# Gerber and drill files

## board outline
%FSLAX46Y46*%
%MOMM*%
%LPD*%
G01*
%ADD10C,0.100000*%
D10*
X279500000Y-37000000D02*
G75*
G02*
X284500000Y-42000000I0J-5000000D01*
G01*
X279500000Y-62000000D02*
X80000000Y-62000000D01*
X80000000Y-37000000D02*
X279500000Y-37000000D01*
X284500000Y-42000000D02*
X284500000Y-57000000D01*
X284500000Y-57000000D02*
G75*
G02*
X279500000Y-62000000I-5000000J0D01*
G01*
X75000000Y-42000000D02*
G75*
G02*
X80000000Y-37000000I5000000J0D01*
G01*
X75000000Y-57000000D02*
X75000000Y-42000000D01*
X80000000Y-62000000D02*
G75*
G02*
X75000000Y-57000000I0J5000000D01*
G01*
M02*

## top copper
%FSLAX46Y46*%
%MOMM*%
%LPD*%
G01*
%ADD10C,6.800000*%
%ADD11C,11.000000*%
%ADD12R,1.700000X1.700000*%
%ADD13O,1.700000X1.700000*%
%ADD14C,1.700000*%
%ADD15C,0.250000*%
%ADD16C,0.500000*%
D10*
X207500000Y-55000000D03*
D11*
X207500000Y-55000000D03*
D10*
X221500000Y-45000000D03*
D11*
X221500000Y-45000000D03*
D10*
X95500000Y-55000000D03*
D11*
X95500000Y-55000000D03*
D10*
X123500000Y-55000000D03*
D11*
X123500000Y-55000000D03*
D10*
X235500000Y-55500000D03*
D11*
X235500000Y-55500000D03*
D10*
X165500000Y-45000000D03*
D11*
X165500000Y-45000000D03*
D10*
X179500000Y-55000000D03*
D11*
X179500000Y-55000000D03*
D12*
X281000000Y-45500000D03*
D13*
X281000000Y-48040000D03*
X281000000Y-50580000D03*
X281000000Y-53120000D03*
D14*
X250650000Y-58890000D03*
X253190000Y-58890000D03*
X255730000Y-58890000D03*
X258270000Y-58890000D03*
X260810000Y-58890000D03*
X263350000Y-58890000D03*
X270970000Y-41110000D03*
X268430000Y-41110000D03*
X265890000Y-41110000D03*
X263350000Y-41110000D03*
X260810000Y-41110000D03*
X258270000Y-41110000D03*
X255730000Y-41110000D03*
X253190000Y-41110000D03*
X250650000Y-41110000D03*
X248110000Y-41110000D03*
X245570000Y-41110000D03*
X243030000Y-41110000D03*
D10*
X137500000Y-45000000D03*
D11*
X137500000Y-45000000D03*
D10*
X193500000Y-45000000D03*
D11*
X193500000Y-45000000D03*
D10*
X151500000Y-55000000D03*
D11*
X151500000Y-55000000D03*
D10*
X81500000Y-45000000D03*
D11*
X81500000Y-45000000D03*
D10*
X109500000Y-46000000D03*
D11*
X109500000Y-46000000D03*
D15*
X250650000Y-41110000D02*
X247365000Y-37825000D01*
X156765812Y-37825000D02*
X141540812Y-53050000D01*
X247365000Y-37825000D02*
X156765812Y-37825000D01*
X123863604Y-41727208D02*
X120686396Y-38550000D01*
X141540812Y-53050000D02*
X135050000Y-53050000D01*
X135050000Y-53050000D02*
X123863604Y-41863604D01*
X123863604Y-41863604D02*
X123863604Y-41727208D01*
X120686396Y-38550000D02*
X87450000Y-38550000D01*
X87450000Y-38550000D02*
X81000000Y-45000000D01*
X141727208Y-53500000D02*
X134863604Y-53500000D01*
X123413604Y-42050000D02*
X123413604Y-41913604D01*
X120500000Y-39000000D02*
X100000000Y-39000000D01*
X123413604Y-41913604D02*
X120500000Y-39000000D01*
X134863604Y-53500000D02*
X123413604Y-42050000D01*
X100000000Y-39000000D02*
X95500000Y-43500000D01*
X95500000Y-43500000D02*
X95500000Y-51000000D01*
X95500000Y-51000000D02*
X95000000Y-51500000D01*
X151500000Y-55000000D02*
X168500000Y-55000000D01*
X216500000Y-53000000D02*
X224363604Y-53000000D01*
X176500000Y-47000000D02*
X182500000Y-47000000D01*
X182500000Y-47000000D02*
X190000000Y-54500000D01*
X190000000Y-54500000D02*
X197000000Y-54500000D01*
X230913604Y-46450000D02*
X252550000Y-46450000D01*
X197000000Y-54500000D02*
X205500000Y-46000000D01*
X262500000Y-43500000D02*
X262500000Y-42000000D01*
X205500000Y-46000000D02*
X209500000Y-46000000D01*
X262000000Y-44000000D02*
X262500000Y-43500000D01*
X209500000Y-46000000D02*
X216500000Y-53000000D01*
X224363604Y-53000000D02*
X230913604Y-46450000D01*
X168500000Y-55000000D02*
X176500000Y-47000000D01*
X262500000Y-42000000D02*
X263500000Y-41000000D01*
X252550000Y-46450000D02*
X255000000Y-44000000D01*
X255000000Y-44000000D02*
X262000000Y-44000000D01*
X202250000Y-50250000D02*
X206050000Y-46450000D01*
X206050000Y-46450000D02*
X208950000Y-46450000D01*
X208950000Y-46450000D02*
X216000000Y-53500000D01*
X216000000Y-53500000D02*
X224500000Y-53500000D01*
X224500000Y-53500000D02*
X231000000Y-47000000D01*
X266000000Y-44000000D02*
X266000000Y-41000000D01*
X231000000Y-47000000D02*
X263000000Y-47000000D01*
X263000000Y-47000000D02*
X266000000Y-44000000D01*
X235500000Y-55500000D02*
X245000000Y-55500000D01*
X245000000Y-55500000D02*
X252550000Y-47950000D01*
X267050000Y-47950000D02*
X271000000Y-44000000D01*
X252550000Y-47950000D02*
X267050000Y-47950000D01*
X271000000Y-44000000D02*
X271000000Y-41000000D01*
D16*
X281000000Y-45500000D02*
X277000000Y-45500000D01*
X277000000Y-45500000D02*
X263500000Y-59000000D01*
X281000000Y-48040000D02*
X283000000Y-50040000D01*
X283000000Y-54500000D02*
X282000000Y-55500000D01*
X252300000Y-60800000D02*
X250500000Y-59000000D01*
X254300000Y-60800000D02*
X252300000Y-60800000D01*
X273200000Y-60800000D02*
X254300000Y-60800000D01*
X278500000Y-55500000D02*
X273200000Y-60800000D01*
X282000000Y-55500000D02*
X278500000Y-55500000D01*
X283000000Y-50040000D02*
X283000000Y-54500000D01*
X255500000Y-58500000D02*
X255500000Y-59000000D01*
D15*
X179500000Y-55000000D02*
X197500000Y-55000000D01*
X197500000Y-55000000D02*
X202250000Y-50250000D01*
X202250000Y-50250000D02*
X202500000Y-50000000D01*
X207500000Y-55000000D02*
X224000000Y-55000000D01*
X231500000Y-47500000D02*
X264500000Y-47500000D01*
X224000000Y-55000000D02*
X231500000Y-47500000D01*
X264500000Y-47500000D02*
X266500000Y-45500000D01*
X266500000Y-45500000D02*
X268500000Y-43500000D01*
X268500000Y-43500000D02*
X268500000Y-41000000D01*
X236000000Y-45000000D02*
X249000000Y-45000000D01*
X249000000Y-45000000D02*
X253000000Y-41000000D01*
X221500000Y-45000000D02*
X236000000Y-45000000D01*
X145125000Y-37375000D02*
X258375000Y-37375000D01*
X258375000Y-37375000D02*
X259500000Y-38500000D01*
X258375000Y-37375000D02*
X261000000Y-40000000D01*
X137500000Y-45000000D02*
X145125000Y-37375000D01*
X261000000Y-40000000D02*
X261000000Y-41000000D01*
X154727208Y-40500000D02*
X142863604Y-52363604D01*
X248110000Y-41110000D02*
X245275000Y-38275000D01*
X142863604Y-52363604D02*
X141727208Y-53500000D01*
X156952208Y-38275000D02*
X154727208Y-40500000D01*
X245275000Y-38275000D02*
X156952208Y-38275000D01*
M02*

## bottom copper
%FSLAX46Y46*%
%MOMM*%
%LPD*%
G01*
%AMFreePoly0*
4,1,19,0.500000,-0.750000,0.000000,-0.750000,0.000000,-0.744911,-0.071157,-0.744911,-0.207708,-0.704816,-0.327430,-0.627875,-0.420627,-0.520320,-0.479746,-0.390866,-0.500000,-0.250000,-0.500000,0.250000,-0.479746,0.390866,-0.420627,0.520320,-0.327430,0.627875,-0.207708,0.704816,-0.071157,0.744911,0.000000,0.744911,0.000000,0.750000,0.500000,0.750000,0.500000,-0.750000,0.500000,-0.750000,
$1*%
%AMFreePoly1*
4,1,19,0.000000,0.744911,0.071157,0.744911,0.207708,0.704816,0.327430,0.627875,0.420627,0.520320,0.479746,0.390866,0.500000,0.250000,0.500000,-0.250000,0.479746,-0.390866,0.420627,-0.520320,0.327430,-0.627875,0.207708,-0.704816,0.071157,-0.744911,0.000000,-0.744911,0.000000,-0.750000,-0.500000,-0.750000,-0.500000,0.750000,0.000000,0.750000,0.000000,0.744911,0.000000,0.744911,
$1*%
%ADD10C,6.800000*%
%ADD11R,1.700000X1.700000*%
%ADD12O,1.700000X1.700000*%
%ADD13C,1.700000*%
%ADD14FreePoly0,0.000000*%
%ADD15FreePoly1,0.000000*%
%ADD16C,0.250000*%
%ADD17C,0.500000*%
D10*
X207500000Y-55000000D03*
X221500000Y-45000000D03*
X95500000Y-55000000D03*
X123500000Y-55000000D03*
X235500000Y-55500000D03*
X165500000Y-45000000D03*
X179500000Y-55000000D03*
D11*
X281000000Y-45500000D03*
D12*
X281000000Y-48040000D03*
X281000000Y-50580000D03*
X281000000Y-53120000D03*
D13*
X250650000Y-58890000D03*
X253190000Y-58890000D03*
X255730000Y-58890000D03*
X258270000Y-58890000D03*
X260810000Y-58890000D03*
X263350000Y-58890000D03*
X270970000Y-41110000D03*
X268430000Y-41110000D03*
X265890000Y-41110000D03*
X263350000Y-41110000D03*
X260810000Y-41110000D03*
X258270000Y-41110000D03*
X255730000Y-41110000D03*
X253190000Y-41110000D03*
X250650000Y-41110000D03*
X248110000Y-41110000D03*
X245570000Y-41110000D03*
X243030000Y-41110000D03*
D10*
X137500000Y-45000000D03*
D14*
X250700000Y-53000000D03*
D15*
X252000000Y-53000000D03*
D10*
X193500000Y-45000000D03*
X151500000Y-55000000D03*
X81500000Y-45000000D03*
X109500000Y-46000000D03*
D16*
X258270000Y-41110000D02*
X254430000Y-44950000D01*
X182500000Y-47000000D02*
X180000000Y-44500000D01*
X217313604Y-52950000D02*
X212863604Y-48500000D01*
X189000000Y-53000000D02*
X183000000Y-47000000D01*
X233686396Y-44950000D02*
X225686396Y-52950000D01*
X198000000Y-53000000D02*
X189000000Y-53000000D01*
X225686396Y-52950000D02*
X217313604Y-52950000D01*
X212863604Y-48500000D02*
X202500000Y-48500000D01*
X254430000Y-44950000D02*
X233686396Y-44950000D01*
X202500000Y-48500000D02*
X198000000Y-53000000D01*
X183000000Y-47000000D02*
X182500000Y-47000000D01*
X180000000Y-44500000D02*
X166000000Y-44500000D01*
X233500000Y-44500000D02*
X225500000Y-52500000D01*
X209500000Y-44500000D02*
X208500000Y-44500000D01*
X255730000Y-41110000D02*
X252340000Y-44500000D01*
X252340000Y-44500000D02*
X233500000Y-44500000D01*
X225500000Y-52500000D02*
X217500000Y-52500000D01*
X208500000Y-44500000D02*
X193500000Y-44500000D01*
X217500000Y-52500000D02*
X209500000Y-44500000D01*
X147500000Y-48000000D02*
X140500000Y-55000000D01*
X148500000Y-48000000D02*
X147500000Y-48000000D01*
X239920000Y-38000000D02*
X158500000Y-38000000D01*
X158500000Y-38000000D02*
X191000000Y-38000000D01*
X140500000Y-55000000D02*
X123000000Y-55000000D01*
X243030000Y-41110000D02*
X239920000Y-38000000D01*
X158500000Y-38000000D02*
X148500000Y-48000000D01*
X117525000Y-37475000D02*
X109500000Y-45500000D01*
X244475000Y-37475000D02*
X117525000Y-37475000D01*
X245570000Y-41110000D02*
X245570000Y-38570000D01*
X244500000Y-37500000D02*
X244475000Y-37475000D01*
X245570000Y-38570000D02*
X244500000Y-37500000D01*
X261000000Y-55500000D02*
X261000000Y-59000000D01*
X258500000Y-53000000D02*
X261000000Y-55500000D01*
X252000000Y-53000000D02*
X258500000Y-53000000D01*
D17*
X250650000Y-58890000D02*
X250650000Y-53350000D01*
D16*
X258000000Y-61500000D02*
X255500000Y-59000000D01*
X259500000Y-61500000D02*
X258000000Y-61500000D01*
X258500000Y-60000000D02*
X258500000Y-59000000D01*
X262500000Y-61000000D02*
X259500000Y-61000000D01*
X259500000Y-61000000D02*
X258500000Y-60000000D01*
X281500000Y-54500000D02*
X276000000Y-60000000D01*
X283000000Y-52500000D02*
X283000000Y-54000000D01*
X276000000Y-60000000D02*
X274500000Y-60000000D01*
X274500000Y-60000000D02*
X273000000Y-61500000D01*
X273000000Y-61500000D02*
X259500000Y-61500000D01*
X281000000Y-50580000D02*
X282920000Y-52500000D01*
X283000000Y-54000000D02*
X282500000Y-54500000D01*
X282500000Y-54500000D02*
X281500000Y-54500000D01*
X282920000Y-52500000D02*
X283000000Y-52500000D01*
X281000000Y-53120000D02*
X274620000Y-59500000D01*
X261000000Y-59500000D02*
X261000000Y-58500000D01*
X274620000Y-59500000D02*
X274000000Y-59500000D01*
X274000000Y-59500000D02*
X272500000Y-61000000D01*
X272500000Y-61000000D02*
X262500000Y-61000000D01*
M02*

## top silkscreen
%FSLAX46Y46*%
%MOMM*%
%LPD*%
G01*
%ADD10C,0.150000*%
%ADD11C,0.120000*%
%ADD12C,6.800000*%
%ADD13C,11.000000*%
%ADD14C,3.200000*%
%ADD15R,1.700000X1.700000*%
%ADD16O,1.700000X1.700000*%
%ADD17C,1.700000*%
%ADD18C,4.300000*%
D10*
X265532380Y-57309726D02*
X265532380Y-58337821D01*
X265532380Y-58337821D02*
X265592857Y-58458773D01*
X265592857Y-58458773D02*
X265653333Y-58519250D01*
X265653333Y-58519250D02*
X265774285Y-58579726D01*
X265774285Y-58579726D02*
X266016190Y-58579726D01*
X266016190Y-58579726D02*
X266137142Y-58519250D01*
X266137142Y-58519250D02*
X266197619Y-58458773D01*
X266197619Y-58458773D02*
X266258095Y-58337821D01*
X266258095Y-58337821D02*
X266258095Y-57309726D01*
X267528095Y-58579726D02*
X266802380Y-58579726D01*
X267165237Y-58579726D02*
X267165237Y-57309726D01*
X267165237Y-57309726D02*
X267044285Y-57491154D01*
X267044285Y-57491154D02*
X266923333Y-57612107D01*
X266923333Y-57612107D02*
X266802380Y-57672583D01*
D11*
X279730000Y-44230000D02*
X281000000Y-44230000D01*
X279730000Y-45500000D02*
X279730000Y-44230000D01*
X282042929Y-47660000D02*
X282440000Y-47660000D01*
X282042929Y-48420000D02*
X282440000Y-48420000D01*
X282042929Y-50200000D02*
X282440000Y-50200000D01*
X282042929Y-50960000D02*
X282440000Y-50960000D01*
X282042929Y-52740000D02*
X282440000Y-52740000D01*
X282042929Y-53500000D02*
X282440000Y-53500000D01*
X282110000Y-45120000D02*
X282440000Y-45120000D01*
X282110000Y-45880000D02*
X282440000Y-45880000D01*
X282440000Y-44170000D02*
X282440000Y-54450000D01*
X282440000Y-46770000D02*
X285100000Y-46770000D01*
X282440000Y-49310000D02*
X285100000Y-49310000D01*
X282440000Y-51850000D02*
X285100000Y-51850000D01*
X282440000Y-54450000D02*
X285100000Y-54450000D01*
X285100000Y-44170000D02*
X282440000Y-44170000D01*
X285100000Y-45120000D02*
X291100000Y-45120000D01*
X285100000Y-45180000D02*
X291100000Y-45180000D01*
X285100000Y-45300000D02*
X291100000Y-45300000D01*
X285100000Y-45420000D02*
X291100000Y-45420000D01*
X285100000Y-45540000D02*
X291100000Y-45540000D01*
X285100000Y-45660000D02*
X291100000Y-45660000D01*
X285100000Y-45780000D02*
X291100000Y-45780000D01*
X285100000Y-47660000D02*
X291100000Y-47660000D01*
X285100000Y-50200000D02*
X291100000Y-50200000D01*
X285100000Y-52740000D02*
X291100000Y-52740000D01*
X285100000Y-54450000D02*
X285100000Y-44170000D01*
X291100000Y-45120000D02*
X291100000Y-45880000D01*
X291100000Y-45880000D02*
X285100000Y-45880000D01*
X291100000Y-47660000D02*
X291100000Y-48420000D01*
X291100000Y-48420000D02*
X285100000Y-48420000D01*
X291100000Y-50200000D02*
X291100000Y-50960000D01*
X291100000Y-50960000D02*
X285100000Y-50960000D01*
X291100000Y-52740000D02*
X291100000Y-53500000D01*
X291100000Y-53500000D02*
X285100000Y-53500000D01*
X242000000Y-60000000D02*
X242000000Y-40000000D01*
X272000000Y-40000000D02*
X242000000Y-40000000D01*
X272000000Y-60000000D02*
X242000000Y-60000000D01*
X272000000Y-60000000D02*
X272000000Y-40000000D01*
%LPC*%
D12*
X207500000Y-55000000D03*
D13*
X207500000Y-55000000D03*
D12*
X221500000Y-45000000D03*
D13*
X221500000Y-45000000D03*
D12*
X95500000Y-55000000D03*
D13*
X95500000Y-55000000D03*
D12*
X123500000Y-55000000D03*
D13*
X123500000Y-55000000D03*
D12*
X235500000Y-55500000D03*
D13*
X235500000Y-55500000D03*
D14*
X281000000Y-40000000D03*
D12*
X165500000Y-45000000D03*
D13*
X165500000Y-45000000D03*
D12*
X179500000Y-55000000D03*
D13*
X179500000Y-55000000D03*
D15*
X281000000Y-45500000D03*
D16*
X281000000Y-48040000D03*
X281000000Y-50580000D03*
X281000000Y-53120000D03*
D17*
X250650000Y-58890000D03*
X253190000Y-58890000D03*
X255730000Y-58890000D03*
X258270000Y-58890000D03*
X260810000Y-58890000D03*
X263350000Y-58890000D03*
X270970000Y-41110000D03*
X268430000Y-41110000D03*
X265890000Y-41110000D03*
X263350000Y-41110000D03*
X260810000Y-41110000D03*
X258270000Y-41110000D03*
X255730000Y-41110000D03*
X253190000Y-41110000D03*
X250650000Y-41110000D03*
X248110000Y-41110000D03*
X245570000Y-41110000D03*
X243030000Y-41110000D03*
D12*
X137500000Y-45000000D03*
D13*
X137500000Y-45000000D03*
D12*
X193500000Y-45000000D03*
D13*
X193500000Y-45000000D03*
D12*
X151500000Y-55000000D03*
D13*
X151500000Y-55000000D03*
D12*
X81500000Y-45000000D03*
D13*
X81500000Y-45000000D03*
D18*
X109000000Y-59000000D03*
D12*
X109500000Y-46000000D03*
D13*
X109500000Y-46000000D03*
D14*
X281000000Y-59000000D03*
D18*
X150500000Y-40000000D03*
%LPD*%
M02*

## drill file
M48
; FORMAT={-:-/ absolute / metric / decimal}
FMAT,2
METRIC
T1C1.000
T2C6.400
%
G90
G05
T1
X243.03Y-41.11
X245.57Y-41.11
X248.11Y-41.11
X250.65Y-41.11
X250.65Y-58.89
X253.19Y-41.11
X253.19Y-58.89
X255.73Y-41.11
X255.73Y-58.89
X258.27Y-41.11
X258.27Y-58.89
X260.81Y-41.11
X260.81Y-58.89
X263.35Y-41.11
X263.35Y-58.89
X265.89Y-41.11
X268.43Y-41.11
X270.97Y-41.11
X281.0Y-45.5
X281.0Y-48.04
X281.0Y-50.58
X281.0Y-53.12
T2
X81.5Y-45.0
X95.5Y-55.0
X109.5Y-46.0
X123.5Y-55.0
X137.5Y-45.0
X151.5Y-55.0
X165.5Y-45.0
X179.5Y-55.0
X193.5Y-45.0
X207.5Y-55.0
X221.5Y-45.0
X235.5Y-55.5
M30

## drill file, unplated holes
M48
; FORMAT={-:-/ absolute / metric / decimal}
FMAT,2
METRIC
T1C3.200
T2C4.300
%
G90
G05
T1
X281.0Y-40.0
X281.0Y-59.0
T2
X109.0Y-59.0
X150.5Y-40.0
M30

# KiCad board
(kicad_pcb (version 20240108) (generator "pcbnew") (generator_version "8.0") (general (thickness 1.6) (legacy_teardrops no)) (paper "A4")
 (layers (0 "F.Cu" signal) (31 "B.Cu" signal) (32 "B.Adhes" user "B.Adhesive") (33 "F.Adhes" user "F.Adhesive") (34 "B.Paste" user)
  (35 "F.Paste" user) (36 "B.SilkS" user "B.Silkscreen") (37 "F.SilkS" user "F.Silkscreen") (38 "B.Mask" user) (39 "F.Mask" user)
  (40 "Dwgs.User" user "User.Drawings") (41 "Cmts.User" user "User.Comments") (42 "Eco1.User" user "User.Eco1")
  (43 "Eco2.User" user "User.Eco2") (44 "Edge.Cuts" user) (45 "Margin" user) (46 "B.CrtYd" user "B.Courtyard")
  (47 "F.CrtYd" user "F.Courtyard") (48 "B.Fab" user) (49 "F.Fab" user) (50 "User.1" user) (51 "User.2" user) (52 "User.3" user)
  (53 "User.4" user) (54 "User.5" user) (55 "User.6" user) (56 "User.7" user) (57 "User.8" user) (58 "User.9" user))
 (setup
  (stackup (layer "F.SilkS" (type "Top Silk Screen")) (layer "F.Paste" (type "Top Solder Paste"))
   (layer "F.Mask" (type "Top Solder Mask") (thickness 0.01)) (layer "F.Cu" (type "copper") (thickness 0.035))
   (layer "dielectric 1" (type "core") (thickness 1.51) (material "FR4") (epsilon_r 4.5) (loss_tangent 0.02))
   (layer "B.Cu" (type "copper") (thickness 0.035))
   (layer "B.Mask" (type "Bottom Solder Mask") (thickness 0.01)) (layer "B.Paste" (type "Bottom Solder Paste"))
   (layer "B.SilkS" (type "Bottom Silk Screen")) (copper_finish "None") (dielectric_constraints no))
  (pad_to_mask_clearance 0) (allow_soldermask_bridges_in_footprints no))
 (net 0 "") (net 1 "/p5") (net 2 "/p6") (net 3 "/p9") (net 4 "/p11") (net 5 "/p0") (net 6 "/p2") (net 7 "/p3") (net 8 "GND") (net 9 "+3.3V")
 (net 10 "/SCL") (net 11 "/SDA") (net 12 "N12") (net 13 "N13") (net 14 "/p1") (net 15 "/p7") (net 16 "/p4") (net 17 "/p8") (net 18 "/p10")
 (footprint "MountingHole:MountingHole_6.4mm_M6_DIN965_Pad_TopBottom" (layer "F.Cu") (at 207.5 55 90)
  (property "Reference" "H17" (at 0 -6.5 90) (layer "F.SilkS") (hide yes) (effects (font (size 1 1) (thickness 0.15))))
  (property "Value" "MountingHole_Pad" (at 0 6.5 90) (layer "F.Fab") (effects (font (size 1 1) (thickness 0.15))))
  (pad "" connect circle (at 0 0 90) (size 11 11) (layers "B.Mask" "Rescue"))
  (pad "1" thru_hole circle (at 0 0 90) (size 6.8 6.8) (drill 6.4) (layers "*.Cu" "*.Mask") (remove_unused_layers no) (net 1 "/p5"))
  (pad "1" connect circle (at 0 0 90) (size 11 11) (layers "F.Cu" "F.Mask") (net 1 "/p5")))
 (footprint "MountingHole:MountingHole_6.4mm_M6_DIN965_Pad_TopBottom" (layer "F.Cu") (at 221.5 45 90)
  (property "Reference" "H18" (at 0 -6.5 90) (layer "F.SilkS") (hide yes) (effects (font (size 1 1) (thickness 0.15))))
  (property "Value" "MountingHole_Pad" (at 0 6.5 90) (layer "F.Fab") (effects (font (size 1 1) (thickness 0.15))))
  (pad "" connect circle (at 0 0 90) (size 11 11) (layers "B.Mask" "Rescue"))
  (pad "1" thru_hole circle (at 0 0 90) (size 6.8 6.8) (drill 6.4) (layers "*.Cu" "*.Mask") (remove_unused_layers no) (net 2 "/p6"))
  (pad "1" connect circle (at 0 0 90) (size 11 11) (layers "F.Cu" "F.Mask") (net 2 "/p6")))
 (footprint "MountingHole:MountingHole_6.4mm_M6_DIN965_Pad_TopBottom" (layer "F.Cu") (at 95.5 55)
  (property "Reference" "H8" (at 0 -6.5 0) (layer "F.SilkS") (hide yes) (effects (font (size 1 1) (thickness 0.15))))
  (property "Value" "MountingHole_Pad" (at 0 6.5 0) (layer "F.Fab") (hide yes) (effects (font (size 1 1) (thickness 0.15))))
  (pad "" connect circle (at 0 0) (size 11 11) (layers "B.Mask" "Rescue"))
  (pad "1" thru_hole circle (at 0 0) (size 6.8 6.8) (drill 6.4) (layers "*.Cu" "*.Mask") (remove_unused_layers no) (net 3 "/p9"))
  (pad "1" connect circle (at 0 0) (size 11 11) (layers "F.Cu" "F.Mask") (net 3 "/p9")))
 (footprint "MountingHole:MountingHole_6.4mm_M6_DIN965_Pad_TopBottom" (layer "F.Cu") (at 123.5 55 90)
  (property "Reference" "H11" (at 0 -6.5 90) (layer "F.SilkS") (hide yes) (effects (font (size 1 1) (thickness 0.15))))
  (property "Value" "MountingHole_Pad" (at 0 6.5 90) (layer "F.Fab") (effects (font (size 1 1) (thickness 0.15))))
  (pad "" connect circle (at 0 0 90) (size 11 11) (layers "B.Mask" "Rescue"))
  (pad "1" thru_hole circle (at 0 0 90) (size 6.8 6.8) (drill 6.4) (layers "*.Cu" "*.Mask") (remove_unused_layers no) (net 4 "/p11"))
  (pad "1" connect circle (at 0 0 90) (size 11 11) (layers "F.Cu" "F.Mask") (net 4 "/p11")))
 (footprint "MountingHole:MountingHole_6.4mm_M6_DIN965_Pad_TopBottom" (layer "F.Cu") (at 235.5 55.5 90)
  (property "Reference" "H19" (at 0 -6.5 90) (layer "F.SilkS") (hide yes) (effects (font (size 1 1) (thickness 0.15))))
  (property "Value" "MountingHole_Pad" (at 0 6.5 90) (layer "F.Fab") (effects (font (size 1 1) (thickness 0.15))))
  (pad "" connect circle (at 0 0 90) (size 11 11) (layers "B.Mask" "Rescue"))
  (pad "1" thru_hole circle (at 0 0 90) (size 6.8 6.8) (drill 6.4) (layers "*.Cu" "*.Mask") (remove_unused_layers no) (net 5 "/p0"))
  (pad "1" connect circle (at 0 0 90) (size 11 11) (layers "F.Cu" "F.Mask") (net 5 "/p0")))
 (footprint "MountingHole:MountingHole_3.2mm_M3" (layer "F.Cu") (at 283.7475 40.08 -90)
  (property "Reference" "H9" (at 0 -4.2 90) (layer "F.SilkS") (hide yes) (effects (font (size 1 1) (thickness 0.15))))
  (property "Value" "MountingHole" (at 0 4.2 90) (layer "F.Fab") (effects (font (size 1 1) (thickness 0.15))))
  (pad "" np_thru_hole circle (at -0.08 2.7475 270) (size 3.2 3.2) (drill 3.2) (layers "F&B.Cu" "*.Mask")))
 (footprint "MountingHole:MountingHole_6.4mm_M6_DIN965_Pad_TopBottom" (layer "F.Cu") (at 165.5 45 90)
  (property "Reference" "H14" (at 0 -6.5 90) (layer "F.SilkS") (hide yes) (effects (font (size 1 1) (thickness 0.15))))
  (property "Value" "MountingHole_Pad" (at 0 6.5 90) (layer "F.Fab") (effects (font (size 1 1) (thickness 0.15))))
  (pad "" connect circle (at 0 0 90) (size 11 11) (layers "B.Mask" "Rescue"))
  (pad "1" thru_hole circle (at 0 0 90) (size 6.8 6.8) (drill 6.4) (layers "*.Cu" "*.Mask") (remove_unused_layers no) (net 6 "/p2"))
  (pad "1" connect circle (at 0 0 90) (size 11 11) (layers "F.Cu" "F.Mask") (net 6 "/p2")))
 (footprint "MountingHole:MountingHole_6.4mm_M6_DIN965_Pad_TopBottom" (layer "F.Cu") (at 179.5 55 90)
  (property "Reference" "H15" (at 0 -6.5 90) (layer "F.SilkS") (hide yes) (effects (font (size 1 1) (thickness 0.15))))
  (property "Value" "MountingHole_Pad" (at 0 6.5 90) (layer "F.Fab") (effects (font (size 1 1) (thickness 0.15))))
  (pad "" connect circle (at 0 0 90) (size 11 11) (layers "B.Mask" "Rescue"))
  (pad "1" thru_hole circle (at 0 0 90) (size 6.8 6.8) (drill 6.4) (layers "*.Cu" "*.Mask") (remove_unused_layers no) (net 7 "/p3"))
  (pad "1" connect circle (at 0 0 90) (size 11 11) (layers "F.Cu" "F.Mask") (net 7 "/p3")))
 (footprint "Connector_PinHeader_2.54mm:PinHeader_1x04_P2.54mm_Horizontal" (layer "F.Cu") (at 281 45.5)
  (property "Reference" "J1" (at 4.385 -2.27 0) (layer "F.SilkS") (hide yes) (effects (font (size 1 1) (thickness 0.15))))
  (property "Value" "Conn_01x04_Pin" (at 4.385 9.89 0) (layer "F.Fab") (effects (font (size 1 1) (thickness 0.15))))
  (fp_line (start -1.27 -1.27) (end 0 -1.27) (stroke (width 0.12) (type solid)) (layer "F.SilkS"))
  (fp_line (start -1.27 0) (end -1.27 -1.27) (stroke (width 0.12) (type solid)) (layer "F.SilkS"))
  (fp_line (start 1.042929 2.16) (end 1.44 2.16) (stroke (width 0.12) (type solid)) (layer "F.SilkS"))
  (fp_line (start 1.042929 2.92) (end 1.44 2.92) (stroke (width 0.12) (type solid)) (layer "F.SilkS"))
  (fp_line (start 1.042929 4.7) (end 1.44 4.7) (stroke (width 0.12) (type solid)) (layer "F.SilkS"))
  (fp_line (start 1.042929 5.46) (end 1.44 5.46) (stroke (width 0.12) (type solid)) (layer "F.SilkS"))
  (fp_line (start 1.042929 7.24) (end 1.44 7.24) (stroke (width 0.12) (type solid)) (layer "F.SilkS"))
  (fp_line (start 1.042929 8) (end 1.44 8) (stroke (width 0.12) (type solid)) (layer "F.SilkS"))
  (fp_line (start 1.11 -0.38) (end 1.44 -0.38) (stroke (width 0.12) (type solid)) (layer "F.SilkS"))
  (fp_line (start 1.11 0.38) (end 1.44 0.38) (stroke (width 0.12) (type solid)) (layer "F.SilkS"))
  (fp_line (start 1.44 -1.33) (end 1.44 8.95) (stroke (width 0.12) (type solid)) (layer "F.SilkS"))
  (fp_line (start 1.44 1.27) (end 4.1 1.27) (stroke (width 0.12) (type solid)) (layer "F.SilkS"))
  (fp_line (start 1.44 3.81) (end 4.1 3.81) (stroke (width 0.12) (type solid)) (layer "F.SilkS"))
  (fp_line (start 1.44 6.35) (end 4.1 6.35) (stroke (width 0.12) (type solid)) (layer "F.SilkS"))
  (fp_line (start 1.44 8.95) (end 4.1 8.95) (stroke (width 0.12) (type solid)) (layer "F.SilkS"))
  (fp_line (start 4.1 -1.33) (end 1.44 -1.33) (stroke (width 0.12) (type solid)) (layer "F.SilkS"))
  (fp_line (start 4.1 -0.38) (end 10.1 -0.38) (stroke (width 0.12) (type solid)) (layer "F.SilkS"))
  (fp_line (start 4.1 -0.32) (end 10.1 -0.32) (stroke (width 0.12) (type solid)) (layer "F.SilkS"))
  (fp_line (start 4.1 -0.2) (end 10.1 -0.2) (stroke (width 0.12) (type solid)) (layer "F.SilkS"))
  (fp_line (start 4.1 -0.08) (end 10.1 -0.08) (stroke (width 0.12) (type solid)) (layer "F.SilkS"))
  (fp_line (start 4.1 0.04) (end 10.1 0.04) (stroke (width 0.12) (type solid)) (layer "F.SilkS"))
  (fp_line (start 4.1 0.16) (end 10.1 0.16) (stroke (width 0.12) (type solid)) (layer "F.SilkS"))
  (fp_line (start 4.1 0.28) (end 10.1 0.28) (stroke (width 0.12) (type solid)) (layer "F.SilkS"))
  (fp_line (start 4.1 2.16) (end 10.1 2.16) (stroke (width 0.12) (type solid)) (layer "F.SilkS"))
  (fp_line (start 4.1 4.7) (end 10.1 4.7) (stroke (width 0.12) (type solid)) (layer "F.SilkS"))
  (fp_line (start 4.1 7.24) (end 10.1 7.24) (stroke (width 0.12) (type solid)) (layer "F.SilkS"))
  (fp_line (start 4.1 8.95) (end 4.1 -1.33) (stroke (width 0.12) (type solid)) (layer "F.SilkS"))
  (fp_line (start 10.1 -0.38) (end 10.1 0.38) (stroke (width 0.12) (type solid)) (layer "F.SilkS"))
  (fp_line (start 10.1 0.38) (end 4.1 0.38) (stroke (width 0.12) (type solid)) (layer "F.SilkS"))
  (fp_line (start 10.1 2.16) (end 10.1 2.92) (stroke (width 0.12) (type solid)) (layer "F.SilkS"))
  (fp_line (start 10.1 2.92) (end 4.1 2.92) (stroke (width 0.12) (type solid)) (layer "F.SilkS"))
  (fp_line (start 10.1 4.7) (end 10.1 5.46) (stroke (width 0.12) (type solid)) (layer "F.SilkS"))
  (fp_line (start 10.1 5.46) (end 4.1 5.46) (stroke (width 0.12) (type solid)) (layer "F.SilkS"))
  (fp_line (start 10.1 7.24) (end 10.1 8) (stroke (width 0.12) (type solid)) (layer "F.SilkS"))
  (fp_line (start 10.1 8) (end 4.1 8) (stroke (width 0.12) (type solid)) (layer "F.SilkS"))
  (pad "1" thru_hole rect (at 0 0) (size 1.7 1.7) (drill 1) (layers "*.Cu" "*.Mask") (remove_unused_layers no) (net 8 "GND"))
  (pad "2" thru_hole oval (at 0 2.54) (size 1.7 1.7) (drill 1) (layers "*.Cu" "*.Mask") (remove_unused_layers no) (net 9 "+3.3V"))
  (pad "3" thru_hole oval (at 0 5.08) (size 1.7 1.7) (drill 1) (layers "*.Cu" "*.Mask") (remove_unused_layers no) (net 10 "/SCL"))
  (pad "4" thru_hole oval (at 0 7.62) (size 1.7 1.7) (drill 1) (layers "*.Cu" "*.Mask") (remove_unused_layers no) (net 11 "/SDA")))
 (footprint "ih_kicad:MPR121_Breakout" (layer "F.Cu") (at 257 50 180)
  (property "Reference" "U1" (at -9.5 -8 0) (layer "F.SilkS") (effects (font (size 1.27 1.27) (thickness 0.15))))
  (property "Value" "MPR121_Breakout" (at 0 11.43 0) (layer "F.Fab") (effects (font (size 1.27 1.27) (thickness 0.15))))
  (fp_line (start 15 -10) (end 15 10) (stroke (width 0.12) (type solid)) (layer "F.SilkS"))
  (fp_line (start -15 10) (end 15 10) (stroke (width 0.12) (type solid)) (layer "F.SilkS"))
  (fp_line (start -15 -10) (end 15 -10) (stroke (width 0.12) (type solid)) (layer "F.SilkS"))
  (fp_line (start -15 -10) (end -15 10) (stroke (width 0.12) (type solid)) (layer "F.SilkS"))
  (pad "1" thru_hole circle (at 6.35 -8.89 180) (size 1.7 1.7) (drill 1) (layers "*.Cu" "*.Mask") (remove_unused_layers no) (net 9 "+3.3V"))
  (pad "2" thru_hole circle (at 3.81 -8.89 180) (size 1.7 1.7) (drill 1) (layers "*.Cu" "*.Mask") (remove_unused_layers no) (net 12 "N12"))
  (pad "3" thru_hole circle (at 1.27 -8.89 180) (size 1.7 1.7) (drill 1) (layers "*.Cu" "*.Mask") (remove_unused_layers no) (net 10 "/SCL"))
  (pad "4" thru_hole circle (at -1.27 -8.89 180) (size 1.7 1.7) (drill 1) (layers "*.Cu" "*.Mask") (remove_unused_layers no) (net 11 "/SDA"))
  (pad "5" thru_hole circle (at -3.81 -8.89 180) (size 1.7 1.7) (drill 1) (layers "*.Cu" "*.Mask") (remove_unused_layers no) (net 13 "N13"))
  (pad "6" thru_hole circle (at -6.35 -8.89 180) (size 1.7 1.7) (drill 1) (layers "*.Cu" "*.Mask") (remove_unused_layers no) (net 8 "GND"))
  (pad "7" thru_hole circle (at -13.97 8.89 180) (size 1.7 1.7) (drill 1) (layers "*.Cu" "*.Mask") (remove_unused_layers no) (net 5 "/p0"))
  (pad "8" thru_hole circle (at -11.43 8.89 180) (size 1.7 1.7) (drill 1) (layers "*.Cu" "*.Mask") (remove_unused_layers no) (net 1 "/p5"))
  (pad "9" thru_hole circle (at -8.89 8.89 180) (size 1.7 1.7) (drill 1) (layers "*.Cu" "*.Mask") (remove_unused_layers no) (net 7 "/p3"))
  (pad "10" thru_hole circle (at -6.35 8.89 180) (size 1.7 1.7) (drill 1) (layers "*.Cu" "*.Mask") (remove_unused_layers no) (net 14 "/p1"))
  (pad "11" thru_hole circle (at -3.81 8.89 180) (size 1.7 1.7) (drill 1) (layers "*.Cu" "*.Mask") (remove_unused_layers no) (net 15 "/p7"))
  (pad "12" thru_hole circle (at -1.27 8.89 180) (size 1.7 1.7) (drill 1) (layers "*.Cu" "*.Mask") (remove_unused_layers no) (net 6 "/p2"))
  (pad "13" thru_hole circle (at 1.27 8.89 180) (size 1.7 1.7) (drill 1) (layers "*.Cu" "*.Mask") (remove_unused_layers no) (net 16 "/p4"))
  (pad "14" thru_hole circle (at 3.81 8.89 180) (size 1.7 1.7) (drill 1) (layers "*.Cu" "*.Mask") (remove_unused_layers no) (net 2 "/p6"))
  (pad "15" thru_hole circle (at 6.35 8.89 180) (size 1.7 1.7) (drill 1) (layers "*.Cu" "*.Mask") (remove_unused_layers no) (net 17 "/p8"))
  (pad "16" thru_hole circle (at 8.89 8.89 180) (size 1.7 1.7) (drill 1) (layers "*.Cu" "*.Mask") (remove_unused_layers no) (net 3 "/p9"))
  (pad "17" thru_hole circle (at 11.43 8.89 180) (size 1.7 1.7) (drill 1) (layers "*.Cu" "*.Mask") (remove_unused_layers no) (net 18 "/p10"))
  (pad "18" thru_hole circle (at 13.97 8.89 180) (size 1.7 1.7) (drill 1) (layers "*.Cu" "*.Mask") (remove_unused_layers no) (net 4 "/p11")))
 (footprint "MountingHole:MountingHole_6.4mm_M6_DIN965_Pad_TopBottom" (layer "F.Cu") (at 137.5 45 90)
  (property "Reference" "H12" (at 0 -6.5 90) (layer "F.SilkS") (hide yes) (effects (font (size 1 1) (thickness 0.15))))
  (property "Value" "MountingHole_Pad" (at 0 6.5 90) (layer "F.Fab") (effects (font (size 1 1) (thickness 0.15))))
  (pad "" connect circle (at 0 0 90) (size 11 11) (layers "B.Mask" "Rescue"))
  (pad "1" thru_hole circle (at 0 0 90) (size 6.8 6.8) (drill 6.4) (layers "*.Cu" "*.Mask") (remove_unused_layers no) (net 15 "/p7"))
  (pad "1" connect circle (at 0 0 90) (size 11 11) (layers "F.Cu" "F.Mask") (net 15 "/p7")))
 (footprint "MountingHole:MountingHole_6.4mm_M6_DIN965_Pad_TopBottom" (layer "F.Cu") (at 193.5 45 90)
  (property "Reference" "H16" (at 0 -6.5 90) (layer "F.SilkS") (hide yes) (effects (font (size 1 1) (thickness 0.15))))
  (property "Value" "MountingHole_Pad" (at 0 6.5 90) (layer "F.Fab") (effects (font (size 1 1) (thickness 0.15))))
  (pad "" connect circle (at 0 0 90) (size 11 11) (layers "B.Mask" "Rescue"))
  (pad "1" thru_hole circle (at 0 0 90) (size 6.8 6.8) (drill 6.4) (layers "*.Cu" "*.Mask") (remove_unused_layers no) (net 16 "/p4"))
  (pad "1" connect circle (at 0 0 90) (size 11 11) (layers "F.Cu" "F.Mask") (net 16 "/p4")))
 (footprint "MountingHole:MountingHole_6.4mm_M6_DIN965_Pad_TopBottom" (layer "F.Cu") (at 151.5 55 90)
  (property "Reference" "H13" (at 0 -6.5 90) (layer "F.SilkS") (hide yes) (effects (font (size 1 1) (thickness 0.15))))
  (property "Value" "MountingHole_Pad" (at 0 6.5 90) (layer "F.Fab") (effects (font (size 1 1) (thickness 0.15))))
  (pad "" connect circle (at 0 0 90) (size 11 11) (layers "B.Mask" "Rescue"))
  (pad "1" thru_hole circle (at 0 0 90) (size 6.8 6.8) (drill 6.4) (layers "*.Cu" "*.Mask") (remove_unused_layers no) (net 14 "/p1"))
  (pad "1" connect circle (at 0 0 90) (size 11 11) (layers "F.Cu" "F.Mask") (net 14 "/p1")))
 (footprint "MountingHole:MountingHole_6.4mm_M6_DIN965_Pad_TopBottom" (layer "F.Cu") (at 81.5 45)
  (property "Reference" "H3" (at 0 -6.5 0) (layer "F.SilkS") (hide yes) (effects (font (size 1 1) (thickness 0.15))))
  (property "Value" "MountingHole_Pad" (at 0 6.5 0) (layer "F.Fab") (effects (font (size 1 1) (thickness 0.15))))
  (pad "" connect circle (at 0 0) (size 11 11) (layers "B.Mask" "Rescue"))
  (pad "1" thru_hole circle (at 0 0) (size 6.8 6.8) (drill 6.4) (layers "*.Cu" "*.Mask") (remove_unused_layers no) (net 17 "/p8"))
  (pad "1" connect circle (at 0 0) (size 11 11) (layers "F.Cu" "F.Mask") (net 17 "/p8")))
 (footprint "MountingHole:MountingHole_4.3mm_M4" (layer "F.Cu") (at 118 97.5)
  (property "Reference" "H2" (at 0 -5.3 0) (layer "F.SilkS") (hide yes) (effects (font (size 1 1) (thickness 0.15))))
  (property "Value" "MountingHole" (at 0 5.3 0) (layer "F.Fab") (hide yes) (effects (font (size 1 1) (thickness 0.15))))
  (pad "" np_thru_hole circle (at -9 -38.5) (size 4.3 4.3) (drill 4.3) (layers "F&B.Cu" "*.Mask")))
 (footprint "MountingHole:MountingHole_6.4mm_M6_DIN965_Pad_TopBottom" (layer "F.Cu") (at 109.5 46)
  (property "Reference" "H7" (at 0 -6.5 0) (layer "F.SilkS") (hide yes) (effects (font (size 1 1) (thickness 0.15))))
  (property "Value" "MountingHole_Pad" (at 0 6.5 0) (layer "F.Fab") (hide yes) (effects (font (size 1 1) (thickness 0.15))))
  (pad "" connect circle (at 0 0) (size 11 11) (layers "B.Mask" "Rescue"))
  (pad "1" thru_hole circle (at 0 0) (size 6.8 6.8) (drill 6.4) (layers "*.Cu" "*.Mask") (remove_unused_layers no) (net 18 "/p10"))
  (pad "1" connect circle (at 0 0) (size 11 11) (layers "F.Cu" "F.Mask") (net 18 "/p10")))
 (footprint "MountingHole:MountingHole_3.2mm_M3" (layer "F.Cu") (at 278.7475 74.58 -90)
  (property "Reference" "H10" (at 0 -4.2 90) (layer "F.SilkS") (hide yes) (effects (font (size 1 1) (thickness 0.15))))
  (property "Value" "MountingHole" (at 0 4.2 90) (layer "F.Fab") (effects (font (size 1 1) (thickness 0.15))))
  (pad "" np_thru_hole circle (at -15.58 -2.2525 270) (size 3.2 3.2) (drill 3.2) (layers "F&B.Cu" "*.Mask")))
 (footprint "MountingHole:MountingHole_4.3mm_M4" (layer "F.Cu") (at 146.5 97.5)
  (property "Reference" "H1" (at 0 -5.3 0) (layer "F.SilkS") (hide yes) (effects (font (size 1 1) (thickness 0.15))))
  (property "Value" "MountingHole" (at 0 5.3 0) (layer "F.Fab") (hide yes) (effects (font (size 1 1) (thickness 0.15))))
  (pad "" np_thru_hole circle (at 4 -57.5) (size 4.3 4.3) (drill 4.3) (layers "F&B.Cu" "*.Mask")))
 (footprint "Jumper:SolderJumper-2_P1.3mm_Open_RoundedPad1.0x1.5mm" (layer "B.Cu") (at 251.35 53)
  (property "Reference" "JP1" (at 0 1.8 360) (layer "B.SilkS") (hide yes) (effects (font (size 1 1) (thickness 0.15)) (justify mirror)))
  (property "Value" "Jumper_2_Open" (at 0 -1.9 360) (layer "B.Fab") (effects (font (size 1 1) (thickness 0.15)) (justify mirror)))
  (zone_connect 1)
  (pad "1" smd custom (at -0.65 0) (size 1 0.5) (layers "B.Cu" "B.Mask") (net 9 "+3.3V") (zone_connect 2) (thermal_bridge_angle 45)
   (options (clearance outline) (anchor rect)) (primitives))
  (pad "2" smd custom (at 0.65 0) (size 1 0.5) (layers "B.Cu" "B.Mask") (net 13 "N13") (zone_connect 2) (thermal_bridge_angle 45)
   (options (clearance outline) (anchor rect)) (primitives)))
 (gr_arc (start 279.5 37) (mid 283.035534 38.464466) (end 284.5 42) (stroke (width 0.1) (type default)) (layer "Edge.Cuts"))
 (gr_line (start 279.5 62) (end 80 62) (stroke (width 0.1) (type default)) (layer "Edge.Cuts"))
 (gr_line (start 80 37) (end 279.5 37) (stroke (width 0.1) (type default)) (layer "Edge.Cuts"))
 (gr_line (start 284.5 42) (end 284.5 57) (stroke (width 0.1) (type default)) (layer "Edge.Cuts"))
 (gr_arc (start 284.5 57) (mid 283.035534 60.535534) (end 279.5 62) (stroke (width 0.1) (type default)) (layer "Edge.Cuts"))
 (gr_arc (start 75 42) (mid 76.464466 38.464466) (end 80 37) (stroke (width 0.1) (type default)) (layer "Edge.Cuts"))
 (gr_line (start 75 57) (end 75 42) (stroke (width 0.1) (type default)) (layer "Edge.Cuts"))
 (gr_arc (start 80 62) (mid 76.464466 60.535534) (end 75 57) (stroke (width 0.1) (type default)) (layer "Edge.Cuts"))
 (segment (start 281 48.04) (end 283 50.04) (width 0.5) (layer "F.Cu") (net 9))
 (segment (start 283 54.5) (end 282 55.5) (width 0.5) (layer "F.Cu") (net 9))
 (segment (start 252.3 60.8) (end 250.5 59) (width 0.5) (layer "F.Cu") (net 9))
 (segment (start 254.3 60.8) (end 252.3 60.8) (width 0.5) (layer "F.Cu") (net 9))
 (segment (start 273.2 60.8) (end 254.3 60.8) (width 0.5) (layer "F.Cu") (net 9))
 (segment (start 278.5 55.5) (end 273.2 60.8) (width 0.5) (layer "F.Cu") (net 9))
 (segment (start 282 55.5) (end 278.5 55.5) (width 0.5) (layer "F.Cu") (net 9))
 (segment (start 283 50.04) (end 283 54.5) (width 0.5) (layer "F.Cu") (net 9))
 (segment (start 250.65 58.89) (end 250.65 53.35) (width 0.5) (layer "B.Cu") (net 9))
 (segment (start 277 45.5) (end 263.5 59) (width 0.5) (layer "F.Cu") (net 8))
 (segment (start 281 45.5) (end 277 45.5) (width 0.5) (layer "F.Cu") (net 8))
 (segment (start 117.525 37.475) (end 109.5 45.5) (width 0.25) (layer "B.Cu") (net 18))
 (segment (start 244.475 37.475) (end 117.525 37.475) (width 0.25) (layer "B.Cu") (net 18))
 (segment (start 245.57 41.11) (end 245.57 38.57) (width 0.25) (layer "B.Cu") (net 18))
 (segment (start 244.5 37.5) (end 244.475 37.475) (width 0.25) (layer "B.Cu") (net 18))
 (segment (start 245.57 38.57) (end 244.5 37.5) (width 0.25) (layer "B.Cu") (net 18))
 (segment (start 267.05 47.95) (end 271 44) (width 0.25) (layer "F.Cu") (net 5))
 (segment (start 271 44) (end 271 41) (width 0.25) (layer "F.Cu") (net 5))
 (segment (start 235.5 55.5) (end 245 55.5) (width 0.25) (layer "F.Cu") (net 5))
 (segment (start 252.55 47.95) (end 267.05 47.95) (width 0.25) (layer "F.Cu") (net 5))
 (segment (start 245 55.5) (end 252.55 47.95) (width 0.25) (layer "F.Cu") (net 5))
 (segment (start 189 53) (end 183 47) (width 0.25) (layer "B.Cu") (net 6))
 (segment (start 182.5 47) (end 180 44.5) (width 0.25) (layer "B.Cu") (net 6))
 (segment (start 183 47) (end 182.5 47) (width 0.25) (layer "B.Cu") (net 6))
 (segment (start 212.863604 48.5) (end 202.5 48.5) (width 0.25) (layer "B.Cu") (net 6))
 (segment (start 202.5 48.5) (end 198 53) (width 0.25) (layer "B.Cu") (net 6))
 (segment (start 225.686396 52.95) (end 217.313604 52.95) (width 0.25) (layer "B.Cu") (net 6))
 (segment (start 198 53) (end 189 53) (width 0.25) (layer "B.Cu") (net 6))
 (segment (start 180 44.5) (end 166 44.5) (width 0.25) (layer "B.Cu") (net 6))
 (segment (start 217.313604 52.95) (end 212.863604 48.5) (width 0.25) (layer "B.Cu") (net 6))
 (segment (start 254.43 44.95) (end 233.686396 44.95) (width 0.25) (layer "B.Cu") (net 6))
 (segment (start 258.27 41.11) (end 254.43 44.95) (width 0.25) (layer "B.Cu") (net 6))
 (segment (start 233.686396 44.95) (end 225.686396 52.95) (width 0.25) (layer "B.Cu") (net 6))
 (segment (start 255.5 58.5) (end 255.5 59) (width 0.5) (layer "F.Cu") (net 10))
 (segment (start 259.5 61.5) (end 258 61.5) (width 0.25) (layer "B.Cu") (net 10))
 (segment (start 281.5 54.5) (end 276 60) (width 0.25) (layer "B.Cu") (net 10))
 (segment (start 283 52.5) (end 283 54) (width 0.25) (layer "B.Cu") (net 10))
 (segment (start 276 60) (end 274.5 60) (width 0.25) (layer "B.Cu") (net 10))
 (segment (start 274.5 60) (end 273 61.5) (width 0.25) (layer "B.Cu") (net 10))
 (segment (start 273 61.5) (end 259.5 61.5) (width 0.25) (layer "B.Cu") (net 10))
 (segment (start 258 61.5) (end 255.5 59) (width 0.25) (layer "B.Cu") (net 10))
 (segment (start 281 50.58) (end 282.92 52.5) (width 0.25) (layer "B.Cu") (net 10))
 (segment (start 283 54) (end 282.5 54.5) (width 0.25) (layer "B.Cu") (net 10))
 (segment (start 282.5 54.5) (end 281.5 54.5) (width 0.25) (layer "B.Cu") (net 10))
 (segment (start 282.92 52.5) (end 283 52.5) (width 0.25) (layer "B.Cu") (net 10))
 (segment (start 281 53.12) (end 274.62 59.5) (width 0.25) (layer "B.Cu") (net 11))
 (segment (start 259.5 61) (end 258.5 60) (width 0.25) (layer "B.Cu") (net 11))
 (segment (start 274.62 59.5) (end 274 59.5) (width 0.25) (layer "B.Cu") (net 11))
 (segment (start 262.5 61) (end 259.5 61) (width 0.25) (layer "B.Cu") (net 11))
 (segment (start 274 59.5) (end 272.5 61) (width 0.25) (layer "B.Cu") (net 11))
 (segment (start 272.5 61) (end 262.5 61) (width 0.25) (layer "B.Cu") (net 11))
 (segment (start 258.5 60) (end 258.5 59) (width 0.25) (layer "B.Cu") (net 11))
 (segment (start 176.5 47) (end 182.5 47) (width 0.25) (layer "F.Cu") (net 14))
 (segment (start 262.5 42) (end 263.5 41) (width 0.25) (layer "F.Cu") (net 14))
 (segment (start 255 44) (end 262 44) (width 0.25) (layer "F.Cu") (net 14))
 (segment (start 252.55 46.45) (end 255 44) (width 0.25) (layer "F.Cu") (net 14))
 (segment (start 230.913604 46.45) (end 252.55 46.45) (width 0.25) (layer "F.Cu") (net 14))
 (segment (start 224.363604 53) (end 230.913604 46.45) (width 0.25) (layer "F.Cu") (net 14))
 (segment (start 209.5 46) (end 216.5 53) (width 0.25) (layer "F.Cu") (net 14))
 (segment (start 182.5 47) (end 190 54.5) (width 0.25) (layer "F.Cu") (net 14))
 (segment (start 262 44) (end 262.5 43.5) (width 0.25) (layer "F.Cu") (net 14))
 (segment (start 205.5 46) (end 209.5 46) (width 0.25) (layer "F.Cu") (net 14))
 (segment (start 168.5 55) (end 176.5 47) (width 0.25) (layer "F.Cu") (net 14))
 (segment (start 151.5 55) (end 168.5 55) (width 0.25) (layer "F.Cu") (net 14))
 (segment (start 262.5 43.5) (end 262.5 42) (width 0.25) (layer "F.Cu") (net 14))
 (segment (start 197 54.5) (end 205.5 46) (width 0.25) (layer "F.Cu") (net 14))
 (segment (start 216.5 53) (end 224.363604 53) (width 0.25) (layer "F.Cu") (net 14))
 (segment (start 190 54.5) (end 197 54.5) (width 0.25) (layer "F.Cu") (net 14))
 (segment (start 179.5 55) (end 197.5 55) (width 0.25) (layer "F.Cu") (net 7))
 (segment (start 202.25 50.25) (end 206.05 46.45) (width 0.25) (layer "F.Cu") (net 7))
 (segment (start 206.05 46.45) (end 208.95 46.45) (width 0.25) (layer "F.Cu") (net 7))
 (segment (start 224.5 53.5) (end 231 47) (width 0.25) (layer "F.Cu") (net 7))
 (segment (start 216 53.5) (end 224.5 53.5) (width 0.25) (layer "F.Cu") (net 7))
 (segment (start 263 47) (end 266 44) (width 0.25) (layer "F.Cu") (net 7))
 (segment (start 197.5 55) (end 202.25 50.25) (width 0.25) (layer "F.Cu") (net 7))
 (segment (start 202.25 50.25) (end 202.5 50) (width 0.25) (layer "F.Cu") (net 7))
 (segment (start 266 44) (end 266 41) (width 0.25) (layer "F.Cu") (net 7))
 (segment (start 208.95 46.45) (end 216 53.5) (width 0.25) (layer "F.Cu") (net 7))
 (segment (start 231 47) (end 263 47) (width 0.25) (layer "F.Cu") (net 7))
 (segment (start 233.5 44.5) (end 225.5 52.5) (width 0.25) (layer "B.Cu") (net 16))
 (segment (start 255.73 41.11) (end 252.34 44.5) (width 0.25) (layer "B.Cu") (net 16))
 (segment (start 209.5 44.5) (end 208.5 44.5) (width 0.25) (layer "B.Cu") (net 16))
 (segment (start 208.5 44.5) (end 193.5 44.5) (width 0.25) (layer "B.Cu") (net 16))
 (segment (start 217.5 52.5) (end 209.5 44.5) (width 0.25) (layer "B.Cu") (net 16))
 (segment (start 225.5 52.5) (end 217.5 52.5) (width 0.25) (layer "B.Cu") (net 16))
 (segment (start 252.34 44.5) (end 233.5 44.5) (width 0.25) (layer "B.Cu") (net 16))
 (segment (start 207.5 55) (end 224 55) (width 0.25) (layer "F.Cu") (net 1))
 (segment (start 231.5 47.5) (end 264.5 47.5) (width 0.25) (layer "F.Cu") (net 1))
 (segment (start 224 55) (end 231.5 47.5) (width 0.25) (layer "F.Cu") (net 1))
 (segment (start 264.5 47.5) (end 266.5 45.5) (width 0.25) (layer "F.Cu") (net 1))
 (segment (start 266.5 45.5) (end 268.5 43.5) (width 0.25) (layer "F.Cu") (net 1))
 (segment (start 268.5 43.5) (end 268.5 41) (width 0.25) (layer "F.Cu") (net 1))
 (segment (start 236 45) (end 249 45) (width 0.25) (layer "F.Cu") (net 2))
 (segment (start 249 45) (end 253 41) (width 0.25) (layer "F.Cu") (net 2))
 (segment (start 221.5 45) (end 236 45) (width 0.25) (layer "F.Cu") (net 2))
 (segment (start 145.125 37.375) (end 258.375 37.375) (width 0.25) (layer "F.Cu") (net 15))
 (segment (start 258.375 37.375) (end 259.5 38.5) (width 0.25) (layer "F.Cu") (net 15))
 (segment (start 258.375 37.375) (end 261 40) (width 0.25) (layer "F.Cu") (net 15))
 (segment (start 137.5 45) (end 145.125 37.375) (width 0.25) (layer "F.Cu") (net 15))
 (segment (start 261 40) (end 261 41) (width 0.25) (layer "F.Cu") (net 15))
 (segment (start 247.365 37.825) (end 156.765812 37.825) (width 0.25) (layer "F.Cu") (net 17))
 (segment (start 250.65 41.11) (end 247.365 37.825) (width 0.25) (layer "F.Cu") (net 17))
 (segment (start 156.765812 37.825) (end 141.540812 53.05) (width 0.25) (layer "F.Cu") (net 17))
 (segment (start 141.540812 53.05) (end 135.05 53.05) (width 0.25) (layer "F.Cu") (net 17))
 (segment (start 123.863604 41.863604) (end 123.863604 41.727208) (width 0.25) (layer "F.Cu") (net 17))
 (segment (start 120.686396 38.55) (end 87.45 38.55) (width 0.25) (layer "F.Cu") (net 17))
 (segment (start 123.863604 41.727208) (end 120.686396 38.55) (width 0.25) (layer "F.Cu") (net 17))
 (segment (start 87.45 38.55) (end 81 45) (width 0.25) (layer "F.Cu") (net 17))
 (segment (start 135.05 53.05) (end 123.863604 41.863604) (width 0.25) (layer "F.Cu") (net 17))
 (segment (start 134.863604 53.5) (end 123.413604 42.05) (width 0.25) (layer "F.Cu") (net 3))
 (segment (start 154.727208 40.5) (end 142.863604 52.363604) (width 0.25) (layer "F.Cu") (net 3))
 (segment (start 95.5 51) (end 95 51.5) (width 0.25) (layer "F.Cu") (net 3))
 (segment (start 95.5 43.5) (end 95.5 51) (width 0.25) (layer "F.Cu") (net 3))
 (segment (start 123.413604 42.05) (end 123.413604 41.913604) (width 0.25) (layer "F.Cu") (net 3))
 (segment (start 248.11 41.11) (end 245.275 38.275) (width 0.25) (layer "F.Cu") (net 3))
 (segment (start 142.863604 52.363604) (end 141.727208 53.5) (width 0.25) (layer "F.Cu") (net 3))
 (segment (start 156.952208 38.275) (end 154.727208 40.5) (width 0.25) (layer "F.Cu") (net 3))
 (segment (start 123.413604 41.913604) (end 120.5 39) (width 0.25) (layer "F.Cu") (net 3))
 (segment (start 120.5 39) (end 100 39) (width 0.25) (layer "F.Cu") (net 3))
 (segment (start 245.275 38.275) (end 156.952208 38.275) (width 0.25) (layer "F.Cu") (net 3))
 (segment (start 141.727208 53.5) (end 134.863604 53.5) (width 0.25) (layer "F.Cu") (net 3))
 (segment (start 100 39) (end 95.5 43.5) (width 0.25) (layer "F.Cu") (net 3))
 (segment (start 140.5 55) (end 123 55) (width 0.25) (layer "B.Cu") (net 4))
 (segment (start 239.92 38) (end 158.5 38) (width 0.25) (layer "B.Cu") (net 4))
 (segment (start 148.5 48) (end 147.5 48) (width 0.25) (layer "B.Cu") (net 4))
 (segment (start 147.5 48) (end 140.5 55) (width 0.25) (layer "B.Cu") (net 4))
 (segment (start 158.5 38) (end 191 38) (width 0.25) (layer "B.Cu") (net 4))
 (segment (start 243.03 41.11) (end 239.92 38) (width 0.25) (layer "B.Cu") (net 4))
 (segment (start 158.5 38) (end 148.5 48) (width 0.25) (layer "B.Cu") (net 4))
 (segment (start 258.5 53) (end 261 55.5) (width 0.25) (layer "B.Cu") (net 13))
 (segment (start 252 53) (end 258.5 53) (width 0.25) (layer "B.Cu") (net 13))
 (segment (start 261 59.5) (end 261 58.5) (width 0.25) (layer "B.Cu") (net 13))
 (segment (start 261 55.5) (end 261 59) (width 0.25) (layer "B.Cu") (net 13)))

